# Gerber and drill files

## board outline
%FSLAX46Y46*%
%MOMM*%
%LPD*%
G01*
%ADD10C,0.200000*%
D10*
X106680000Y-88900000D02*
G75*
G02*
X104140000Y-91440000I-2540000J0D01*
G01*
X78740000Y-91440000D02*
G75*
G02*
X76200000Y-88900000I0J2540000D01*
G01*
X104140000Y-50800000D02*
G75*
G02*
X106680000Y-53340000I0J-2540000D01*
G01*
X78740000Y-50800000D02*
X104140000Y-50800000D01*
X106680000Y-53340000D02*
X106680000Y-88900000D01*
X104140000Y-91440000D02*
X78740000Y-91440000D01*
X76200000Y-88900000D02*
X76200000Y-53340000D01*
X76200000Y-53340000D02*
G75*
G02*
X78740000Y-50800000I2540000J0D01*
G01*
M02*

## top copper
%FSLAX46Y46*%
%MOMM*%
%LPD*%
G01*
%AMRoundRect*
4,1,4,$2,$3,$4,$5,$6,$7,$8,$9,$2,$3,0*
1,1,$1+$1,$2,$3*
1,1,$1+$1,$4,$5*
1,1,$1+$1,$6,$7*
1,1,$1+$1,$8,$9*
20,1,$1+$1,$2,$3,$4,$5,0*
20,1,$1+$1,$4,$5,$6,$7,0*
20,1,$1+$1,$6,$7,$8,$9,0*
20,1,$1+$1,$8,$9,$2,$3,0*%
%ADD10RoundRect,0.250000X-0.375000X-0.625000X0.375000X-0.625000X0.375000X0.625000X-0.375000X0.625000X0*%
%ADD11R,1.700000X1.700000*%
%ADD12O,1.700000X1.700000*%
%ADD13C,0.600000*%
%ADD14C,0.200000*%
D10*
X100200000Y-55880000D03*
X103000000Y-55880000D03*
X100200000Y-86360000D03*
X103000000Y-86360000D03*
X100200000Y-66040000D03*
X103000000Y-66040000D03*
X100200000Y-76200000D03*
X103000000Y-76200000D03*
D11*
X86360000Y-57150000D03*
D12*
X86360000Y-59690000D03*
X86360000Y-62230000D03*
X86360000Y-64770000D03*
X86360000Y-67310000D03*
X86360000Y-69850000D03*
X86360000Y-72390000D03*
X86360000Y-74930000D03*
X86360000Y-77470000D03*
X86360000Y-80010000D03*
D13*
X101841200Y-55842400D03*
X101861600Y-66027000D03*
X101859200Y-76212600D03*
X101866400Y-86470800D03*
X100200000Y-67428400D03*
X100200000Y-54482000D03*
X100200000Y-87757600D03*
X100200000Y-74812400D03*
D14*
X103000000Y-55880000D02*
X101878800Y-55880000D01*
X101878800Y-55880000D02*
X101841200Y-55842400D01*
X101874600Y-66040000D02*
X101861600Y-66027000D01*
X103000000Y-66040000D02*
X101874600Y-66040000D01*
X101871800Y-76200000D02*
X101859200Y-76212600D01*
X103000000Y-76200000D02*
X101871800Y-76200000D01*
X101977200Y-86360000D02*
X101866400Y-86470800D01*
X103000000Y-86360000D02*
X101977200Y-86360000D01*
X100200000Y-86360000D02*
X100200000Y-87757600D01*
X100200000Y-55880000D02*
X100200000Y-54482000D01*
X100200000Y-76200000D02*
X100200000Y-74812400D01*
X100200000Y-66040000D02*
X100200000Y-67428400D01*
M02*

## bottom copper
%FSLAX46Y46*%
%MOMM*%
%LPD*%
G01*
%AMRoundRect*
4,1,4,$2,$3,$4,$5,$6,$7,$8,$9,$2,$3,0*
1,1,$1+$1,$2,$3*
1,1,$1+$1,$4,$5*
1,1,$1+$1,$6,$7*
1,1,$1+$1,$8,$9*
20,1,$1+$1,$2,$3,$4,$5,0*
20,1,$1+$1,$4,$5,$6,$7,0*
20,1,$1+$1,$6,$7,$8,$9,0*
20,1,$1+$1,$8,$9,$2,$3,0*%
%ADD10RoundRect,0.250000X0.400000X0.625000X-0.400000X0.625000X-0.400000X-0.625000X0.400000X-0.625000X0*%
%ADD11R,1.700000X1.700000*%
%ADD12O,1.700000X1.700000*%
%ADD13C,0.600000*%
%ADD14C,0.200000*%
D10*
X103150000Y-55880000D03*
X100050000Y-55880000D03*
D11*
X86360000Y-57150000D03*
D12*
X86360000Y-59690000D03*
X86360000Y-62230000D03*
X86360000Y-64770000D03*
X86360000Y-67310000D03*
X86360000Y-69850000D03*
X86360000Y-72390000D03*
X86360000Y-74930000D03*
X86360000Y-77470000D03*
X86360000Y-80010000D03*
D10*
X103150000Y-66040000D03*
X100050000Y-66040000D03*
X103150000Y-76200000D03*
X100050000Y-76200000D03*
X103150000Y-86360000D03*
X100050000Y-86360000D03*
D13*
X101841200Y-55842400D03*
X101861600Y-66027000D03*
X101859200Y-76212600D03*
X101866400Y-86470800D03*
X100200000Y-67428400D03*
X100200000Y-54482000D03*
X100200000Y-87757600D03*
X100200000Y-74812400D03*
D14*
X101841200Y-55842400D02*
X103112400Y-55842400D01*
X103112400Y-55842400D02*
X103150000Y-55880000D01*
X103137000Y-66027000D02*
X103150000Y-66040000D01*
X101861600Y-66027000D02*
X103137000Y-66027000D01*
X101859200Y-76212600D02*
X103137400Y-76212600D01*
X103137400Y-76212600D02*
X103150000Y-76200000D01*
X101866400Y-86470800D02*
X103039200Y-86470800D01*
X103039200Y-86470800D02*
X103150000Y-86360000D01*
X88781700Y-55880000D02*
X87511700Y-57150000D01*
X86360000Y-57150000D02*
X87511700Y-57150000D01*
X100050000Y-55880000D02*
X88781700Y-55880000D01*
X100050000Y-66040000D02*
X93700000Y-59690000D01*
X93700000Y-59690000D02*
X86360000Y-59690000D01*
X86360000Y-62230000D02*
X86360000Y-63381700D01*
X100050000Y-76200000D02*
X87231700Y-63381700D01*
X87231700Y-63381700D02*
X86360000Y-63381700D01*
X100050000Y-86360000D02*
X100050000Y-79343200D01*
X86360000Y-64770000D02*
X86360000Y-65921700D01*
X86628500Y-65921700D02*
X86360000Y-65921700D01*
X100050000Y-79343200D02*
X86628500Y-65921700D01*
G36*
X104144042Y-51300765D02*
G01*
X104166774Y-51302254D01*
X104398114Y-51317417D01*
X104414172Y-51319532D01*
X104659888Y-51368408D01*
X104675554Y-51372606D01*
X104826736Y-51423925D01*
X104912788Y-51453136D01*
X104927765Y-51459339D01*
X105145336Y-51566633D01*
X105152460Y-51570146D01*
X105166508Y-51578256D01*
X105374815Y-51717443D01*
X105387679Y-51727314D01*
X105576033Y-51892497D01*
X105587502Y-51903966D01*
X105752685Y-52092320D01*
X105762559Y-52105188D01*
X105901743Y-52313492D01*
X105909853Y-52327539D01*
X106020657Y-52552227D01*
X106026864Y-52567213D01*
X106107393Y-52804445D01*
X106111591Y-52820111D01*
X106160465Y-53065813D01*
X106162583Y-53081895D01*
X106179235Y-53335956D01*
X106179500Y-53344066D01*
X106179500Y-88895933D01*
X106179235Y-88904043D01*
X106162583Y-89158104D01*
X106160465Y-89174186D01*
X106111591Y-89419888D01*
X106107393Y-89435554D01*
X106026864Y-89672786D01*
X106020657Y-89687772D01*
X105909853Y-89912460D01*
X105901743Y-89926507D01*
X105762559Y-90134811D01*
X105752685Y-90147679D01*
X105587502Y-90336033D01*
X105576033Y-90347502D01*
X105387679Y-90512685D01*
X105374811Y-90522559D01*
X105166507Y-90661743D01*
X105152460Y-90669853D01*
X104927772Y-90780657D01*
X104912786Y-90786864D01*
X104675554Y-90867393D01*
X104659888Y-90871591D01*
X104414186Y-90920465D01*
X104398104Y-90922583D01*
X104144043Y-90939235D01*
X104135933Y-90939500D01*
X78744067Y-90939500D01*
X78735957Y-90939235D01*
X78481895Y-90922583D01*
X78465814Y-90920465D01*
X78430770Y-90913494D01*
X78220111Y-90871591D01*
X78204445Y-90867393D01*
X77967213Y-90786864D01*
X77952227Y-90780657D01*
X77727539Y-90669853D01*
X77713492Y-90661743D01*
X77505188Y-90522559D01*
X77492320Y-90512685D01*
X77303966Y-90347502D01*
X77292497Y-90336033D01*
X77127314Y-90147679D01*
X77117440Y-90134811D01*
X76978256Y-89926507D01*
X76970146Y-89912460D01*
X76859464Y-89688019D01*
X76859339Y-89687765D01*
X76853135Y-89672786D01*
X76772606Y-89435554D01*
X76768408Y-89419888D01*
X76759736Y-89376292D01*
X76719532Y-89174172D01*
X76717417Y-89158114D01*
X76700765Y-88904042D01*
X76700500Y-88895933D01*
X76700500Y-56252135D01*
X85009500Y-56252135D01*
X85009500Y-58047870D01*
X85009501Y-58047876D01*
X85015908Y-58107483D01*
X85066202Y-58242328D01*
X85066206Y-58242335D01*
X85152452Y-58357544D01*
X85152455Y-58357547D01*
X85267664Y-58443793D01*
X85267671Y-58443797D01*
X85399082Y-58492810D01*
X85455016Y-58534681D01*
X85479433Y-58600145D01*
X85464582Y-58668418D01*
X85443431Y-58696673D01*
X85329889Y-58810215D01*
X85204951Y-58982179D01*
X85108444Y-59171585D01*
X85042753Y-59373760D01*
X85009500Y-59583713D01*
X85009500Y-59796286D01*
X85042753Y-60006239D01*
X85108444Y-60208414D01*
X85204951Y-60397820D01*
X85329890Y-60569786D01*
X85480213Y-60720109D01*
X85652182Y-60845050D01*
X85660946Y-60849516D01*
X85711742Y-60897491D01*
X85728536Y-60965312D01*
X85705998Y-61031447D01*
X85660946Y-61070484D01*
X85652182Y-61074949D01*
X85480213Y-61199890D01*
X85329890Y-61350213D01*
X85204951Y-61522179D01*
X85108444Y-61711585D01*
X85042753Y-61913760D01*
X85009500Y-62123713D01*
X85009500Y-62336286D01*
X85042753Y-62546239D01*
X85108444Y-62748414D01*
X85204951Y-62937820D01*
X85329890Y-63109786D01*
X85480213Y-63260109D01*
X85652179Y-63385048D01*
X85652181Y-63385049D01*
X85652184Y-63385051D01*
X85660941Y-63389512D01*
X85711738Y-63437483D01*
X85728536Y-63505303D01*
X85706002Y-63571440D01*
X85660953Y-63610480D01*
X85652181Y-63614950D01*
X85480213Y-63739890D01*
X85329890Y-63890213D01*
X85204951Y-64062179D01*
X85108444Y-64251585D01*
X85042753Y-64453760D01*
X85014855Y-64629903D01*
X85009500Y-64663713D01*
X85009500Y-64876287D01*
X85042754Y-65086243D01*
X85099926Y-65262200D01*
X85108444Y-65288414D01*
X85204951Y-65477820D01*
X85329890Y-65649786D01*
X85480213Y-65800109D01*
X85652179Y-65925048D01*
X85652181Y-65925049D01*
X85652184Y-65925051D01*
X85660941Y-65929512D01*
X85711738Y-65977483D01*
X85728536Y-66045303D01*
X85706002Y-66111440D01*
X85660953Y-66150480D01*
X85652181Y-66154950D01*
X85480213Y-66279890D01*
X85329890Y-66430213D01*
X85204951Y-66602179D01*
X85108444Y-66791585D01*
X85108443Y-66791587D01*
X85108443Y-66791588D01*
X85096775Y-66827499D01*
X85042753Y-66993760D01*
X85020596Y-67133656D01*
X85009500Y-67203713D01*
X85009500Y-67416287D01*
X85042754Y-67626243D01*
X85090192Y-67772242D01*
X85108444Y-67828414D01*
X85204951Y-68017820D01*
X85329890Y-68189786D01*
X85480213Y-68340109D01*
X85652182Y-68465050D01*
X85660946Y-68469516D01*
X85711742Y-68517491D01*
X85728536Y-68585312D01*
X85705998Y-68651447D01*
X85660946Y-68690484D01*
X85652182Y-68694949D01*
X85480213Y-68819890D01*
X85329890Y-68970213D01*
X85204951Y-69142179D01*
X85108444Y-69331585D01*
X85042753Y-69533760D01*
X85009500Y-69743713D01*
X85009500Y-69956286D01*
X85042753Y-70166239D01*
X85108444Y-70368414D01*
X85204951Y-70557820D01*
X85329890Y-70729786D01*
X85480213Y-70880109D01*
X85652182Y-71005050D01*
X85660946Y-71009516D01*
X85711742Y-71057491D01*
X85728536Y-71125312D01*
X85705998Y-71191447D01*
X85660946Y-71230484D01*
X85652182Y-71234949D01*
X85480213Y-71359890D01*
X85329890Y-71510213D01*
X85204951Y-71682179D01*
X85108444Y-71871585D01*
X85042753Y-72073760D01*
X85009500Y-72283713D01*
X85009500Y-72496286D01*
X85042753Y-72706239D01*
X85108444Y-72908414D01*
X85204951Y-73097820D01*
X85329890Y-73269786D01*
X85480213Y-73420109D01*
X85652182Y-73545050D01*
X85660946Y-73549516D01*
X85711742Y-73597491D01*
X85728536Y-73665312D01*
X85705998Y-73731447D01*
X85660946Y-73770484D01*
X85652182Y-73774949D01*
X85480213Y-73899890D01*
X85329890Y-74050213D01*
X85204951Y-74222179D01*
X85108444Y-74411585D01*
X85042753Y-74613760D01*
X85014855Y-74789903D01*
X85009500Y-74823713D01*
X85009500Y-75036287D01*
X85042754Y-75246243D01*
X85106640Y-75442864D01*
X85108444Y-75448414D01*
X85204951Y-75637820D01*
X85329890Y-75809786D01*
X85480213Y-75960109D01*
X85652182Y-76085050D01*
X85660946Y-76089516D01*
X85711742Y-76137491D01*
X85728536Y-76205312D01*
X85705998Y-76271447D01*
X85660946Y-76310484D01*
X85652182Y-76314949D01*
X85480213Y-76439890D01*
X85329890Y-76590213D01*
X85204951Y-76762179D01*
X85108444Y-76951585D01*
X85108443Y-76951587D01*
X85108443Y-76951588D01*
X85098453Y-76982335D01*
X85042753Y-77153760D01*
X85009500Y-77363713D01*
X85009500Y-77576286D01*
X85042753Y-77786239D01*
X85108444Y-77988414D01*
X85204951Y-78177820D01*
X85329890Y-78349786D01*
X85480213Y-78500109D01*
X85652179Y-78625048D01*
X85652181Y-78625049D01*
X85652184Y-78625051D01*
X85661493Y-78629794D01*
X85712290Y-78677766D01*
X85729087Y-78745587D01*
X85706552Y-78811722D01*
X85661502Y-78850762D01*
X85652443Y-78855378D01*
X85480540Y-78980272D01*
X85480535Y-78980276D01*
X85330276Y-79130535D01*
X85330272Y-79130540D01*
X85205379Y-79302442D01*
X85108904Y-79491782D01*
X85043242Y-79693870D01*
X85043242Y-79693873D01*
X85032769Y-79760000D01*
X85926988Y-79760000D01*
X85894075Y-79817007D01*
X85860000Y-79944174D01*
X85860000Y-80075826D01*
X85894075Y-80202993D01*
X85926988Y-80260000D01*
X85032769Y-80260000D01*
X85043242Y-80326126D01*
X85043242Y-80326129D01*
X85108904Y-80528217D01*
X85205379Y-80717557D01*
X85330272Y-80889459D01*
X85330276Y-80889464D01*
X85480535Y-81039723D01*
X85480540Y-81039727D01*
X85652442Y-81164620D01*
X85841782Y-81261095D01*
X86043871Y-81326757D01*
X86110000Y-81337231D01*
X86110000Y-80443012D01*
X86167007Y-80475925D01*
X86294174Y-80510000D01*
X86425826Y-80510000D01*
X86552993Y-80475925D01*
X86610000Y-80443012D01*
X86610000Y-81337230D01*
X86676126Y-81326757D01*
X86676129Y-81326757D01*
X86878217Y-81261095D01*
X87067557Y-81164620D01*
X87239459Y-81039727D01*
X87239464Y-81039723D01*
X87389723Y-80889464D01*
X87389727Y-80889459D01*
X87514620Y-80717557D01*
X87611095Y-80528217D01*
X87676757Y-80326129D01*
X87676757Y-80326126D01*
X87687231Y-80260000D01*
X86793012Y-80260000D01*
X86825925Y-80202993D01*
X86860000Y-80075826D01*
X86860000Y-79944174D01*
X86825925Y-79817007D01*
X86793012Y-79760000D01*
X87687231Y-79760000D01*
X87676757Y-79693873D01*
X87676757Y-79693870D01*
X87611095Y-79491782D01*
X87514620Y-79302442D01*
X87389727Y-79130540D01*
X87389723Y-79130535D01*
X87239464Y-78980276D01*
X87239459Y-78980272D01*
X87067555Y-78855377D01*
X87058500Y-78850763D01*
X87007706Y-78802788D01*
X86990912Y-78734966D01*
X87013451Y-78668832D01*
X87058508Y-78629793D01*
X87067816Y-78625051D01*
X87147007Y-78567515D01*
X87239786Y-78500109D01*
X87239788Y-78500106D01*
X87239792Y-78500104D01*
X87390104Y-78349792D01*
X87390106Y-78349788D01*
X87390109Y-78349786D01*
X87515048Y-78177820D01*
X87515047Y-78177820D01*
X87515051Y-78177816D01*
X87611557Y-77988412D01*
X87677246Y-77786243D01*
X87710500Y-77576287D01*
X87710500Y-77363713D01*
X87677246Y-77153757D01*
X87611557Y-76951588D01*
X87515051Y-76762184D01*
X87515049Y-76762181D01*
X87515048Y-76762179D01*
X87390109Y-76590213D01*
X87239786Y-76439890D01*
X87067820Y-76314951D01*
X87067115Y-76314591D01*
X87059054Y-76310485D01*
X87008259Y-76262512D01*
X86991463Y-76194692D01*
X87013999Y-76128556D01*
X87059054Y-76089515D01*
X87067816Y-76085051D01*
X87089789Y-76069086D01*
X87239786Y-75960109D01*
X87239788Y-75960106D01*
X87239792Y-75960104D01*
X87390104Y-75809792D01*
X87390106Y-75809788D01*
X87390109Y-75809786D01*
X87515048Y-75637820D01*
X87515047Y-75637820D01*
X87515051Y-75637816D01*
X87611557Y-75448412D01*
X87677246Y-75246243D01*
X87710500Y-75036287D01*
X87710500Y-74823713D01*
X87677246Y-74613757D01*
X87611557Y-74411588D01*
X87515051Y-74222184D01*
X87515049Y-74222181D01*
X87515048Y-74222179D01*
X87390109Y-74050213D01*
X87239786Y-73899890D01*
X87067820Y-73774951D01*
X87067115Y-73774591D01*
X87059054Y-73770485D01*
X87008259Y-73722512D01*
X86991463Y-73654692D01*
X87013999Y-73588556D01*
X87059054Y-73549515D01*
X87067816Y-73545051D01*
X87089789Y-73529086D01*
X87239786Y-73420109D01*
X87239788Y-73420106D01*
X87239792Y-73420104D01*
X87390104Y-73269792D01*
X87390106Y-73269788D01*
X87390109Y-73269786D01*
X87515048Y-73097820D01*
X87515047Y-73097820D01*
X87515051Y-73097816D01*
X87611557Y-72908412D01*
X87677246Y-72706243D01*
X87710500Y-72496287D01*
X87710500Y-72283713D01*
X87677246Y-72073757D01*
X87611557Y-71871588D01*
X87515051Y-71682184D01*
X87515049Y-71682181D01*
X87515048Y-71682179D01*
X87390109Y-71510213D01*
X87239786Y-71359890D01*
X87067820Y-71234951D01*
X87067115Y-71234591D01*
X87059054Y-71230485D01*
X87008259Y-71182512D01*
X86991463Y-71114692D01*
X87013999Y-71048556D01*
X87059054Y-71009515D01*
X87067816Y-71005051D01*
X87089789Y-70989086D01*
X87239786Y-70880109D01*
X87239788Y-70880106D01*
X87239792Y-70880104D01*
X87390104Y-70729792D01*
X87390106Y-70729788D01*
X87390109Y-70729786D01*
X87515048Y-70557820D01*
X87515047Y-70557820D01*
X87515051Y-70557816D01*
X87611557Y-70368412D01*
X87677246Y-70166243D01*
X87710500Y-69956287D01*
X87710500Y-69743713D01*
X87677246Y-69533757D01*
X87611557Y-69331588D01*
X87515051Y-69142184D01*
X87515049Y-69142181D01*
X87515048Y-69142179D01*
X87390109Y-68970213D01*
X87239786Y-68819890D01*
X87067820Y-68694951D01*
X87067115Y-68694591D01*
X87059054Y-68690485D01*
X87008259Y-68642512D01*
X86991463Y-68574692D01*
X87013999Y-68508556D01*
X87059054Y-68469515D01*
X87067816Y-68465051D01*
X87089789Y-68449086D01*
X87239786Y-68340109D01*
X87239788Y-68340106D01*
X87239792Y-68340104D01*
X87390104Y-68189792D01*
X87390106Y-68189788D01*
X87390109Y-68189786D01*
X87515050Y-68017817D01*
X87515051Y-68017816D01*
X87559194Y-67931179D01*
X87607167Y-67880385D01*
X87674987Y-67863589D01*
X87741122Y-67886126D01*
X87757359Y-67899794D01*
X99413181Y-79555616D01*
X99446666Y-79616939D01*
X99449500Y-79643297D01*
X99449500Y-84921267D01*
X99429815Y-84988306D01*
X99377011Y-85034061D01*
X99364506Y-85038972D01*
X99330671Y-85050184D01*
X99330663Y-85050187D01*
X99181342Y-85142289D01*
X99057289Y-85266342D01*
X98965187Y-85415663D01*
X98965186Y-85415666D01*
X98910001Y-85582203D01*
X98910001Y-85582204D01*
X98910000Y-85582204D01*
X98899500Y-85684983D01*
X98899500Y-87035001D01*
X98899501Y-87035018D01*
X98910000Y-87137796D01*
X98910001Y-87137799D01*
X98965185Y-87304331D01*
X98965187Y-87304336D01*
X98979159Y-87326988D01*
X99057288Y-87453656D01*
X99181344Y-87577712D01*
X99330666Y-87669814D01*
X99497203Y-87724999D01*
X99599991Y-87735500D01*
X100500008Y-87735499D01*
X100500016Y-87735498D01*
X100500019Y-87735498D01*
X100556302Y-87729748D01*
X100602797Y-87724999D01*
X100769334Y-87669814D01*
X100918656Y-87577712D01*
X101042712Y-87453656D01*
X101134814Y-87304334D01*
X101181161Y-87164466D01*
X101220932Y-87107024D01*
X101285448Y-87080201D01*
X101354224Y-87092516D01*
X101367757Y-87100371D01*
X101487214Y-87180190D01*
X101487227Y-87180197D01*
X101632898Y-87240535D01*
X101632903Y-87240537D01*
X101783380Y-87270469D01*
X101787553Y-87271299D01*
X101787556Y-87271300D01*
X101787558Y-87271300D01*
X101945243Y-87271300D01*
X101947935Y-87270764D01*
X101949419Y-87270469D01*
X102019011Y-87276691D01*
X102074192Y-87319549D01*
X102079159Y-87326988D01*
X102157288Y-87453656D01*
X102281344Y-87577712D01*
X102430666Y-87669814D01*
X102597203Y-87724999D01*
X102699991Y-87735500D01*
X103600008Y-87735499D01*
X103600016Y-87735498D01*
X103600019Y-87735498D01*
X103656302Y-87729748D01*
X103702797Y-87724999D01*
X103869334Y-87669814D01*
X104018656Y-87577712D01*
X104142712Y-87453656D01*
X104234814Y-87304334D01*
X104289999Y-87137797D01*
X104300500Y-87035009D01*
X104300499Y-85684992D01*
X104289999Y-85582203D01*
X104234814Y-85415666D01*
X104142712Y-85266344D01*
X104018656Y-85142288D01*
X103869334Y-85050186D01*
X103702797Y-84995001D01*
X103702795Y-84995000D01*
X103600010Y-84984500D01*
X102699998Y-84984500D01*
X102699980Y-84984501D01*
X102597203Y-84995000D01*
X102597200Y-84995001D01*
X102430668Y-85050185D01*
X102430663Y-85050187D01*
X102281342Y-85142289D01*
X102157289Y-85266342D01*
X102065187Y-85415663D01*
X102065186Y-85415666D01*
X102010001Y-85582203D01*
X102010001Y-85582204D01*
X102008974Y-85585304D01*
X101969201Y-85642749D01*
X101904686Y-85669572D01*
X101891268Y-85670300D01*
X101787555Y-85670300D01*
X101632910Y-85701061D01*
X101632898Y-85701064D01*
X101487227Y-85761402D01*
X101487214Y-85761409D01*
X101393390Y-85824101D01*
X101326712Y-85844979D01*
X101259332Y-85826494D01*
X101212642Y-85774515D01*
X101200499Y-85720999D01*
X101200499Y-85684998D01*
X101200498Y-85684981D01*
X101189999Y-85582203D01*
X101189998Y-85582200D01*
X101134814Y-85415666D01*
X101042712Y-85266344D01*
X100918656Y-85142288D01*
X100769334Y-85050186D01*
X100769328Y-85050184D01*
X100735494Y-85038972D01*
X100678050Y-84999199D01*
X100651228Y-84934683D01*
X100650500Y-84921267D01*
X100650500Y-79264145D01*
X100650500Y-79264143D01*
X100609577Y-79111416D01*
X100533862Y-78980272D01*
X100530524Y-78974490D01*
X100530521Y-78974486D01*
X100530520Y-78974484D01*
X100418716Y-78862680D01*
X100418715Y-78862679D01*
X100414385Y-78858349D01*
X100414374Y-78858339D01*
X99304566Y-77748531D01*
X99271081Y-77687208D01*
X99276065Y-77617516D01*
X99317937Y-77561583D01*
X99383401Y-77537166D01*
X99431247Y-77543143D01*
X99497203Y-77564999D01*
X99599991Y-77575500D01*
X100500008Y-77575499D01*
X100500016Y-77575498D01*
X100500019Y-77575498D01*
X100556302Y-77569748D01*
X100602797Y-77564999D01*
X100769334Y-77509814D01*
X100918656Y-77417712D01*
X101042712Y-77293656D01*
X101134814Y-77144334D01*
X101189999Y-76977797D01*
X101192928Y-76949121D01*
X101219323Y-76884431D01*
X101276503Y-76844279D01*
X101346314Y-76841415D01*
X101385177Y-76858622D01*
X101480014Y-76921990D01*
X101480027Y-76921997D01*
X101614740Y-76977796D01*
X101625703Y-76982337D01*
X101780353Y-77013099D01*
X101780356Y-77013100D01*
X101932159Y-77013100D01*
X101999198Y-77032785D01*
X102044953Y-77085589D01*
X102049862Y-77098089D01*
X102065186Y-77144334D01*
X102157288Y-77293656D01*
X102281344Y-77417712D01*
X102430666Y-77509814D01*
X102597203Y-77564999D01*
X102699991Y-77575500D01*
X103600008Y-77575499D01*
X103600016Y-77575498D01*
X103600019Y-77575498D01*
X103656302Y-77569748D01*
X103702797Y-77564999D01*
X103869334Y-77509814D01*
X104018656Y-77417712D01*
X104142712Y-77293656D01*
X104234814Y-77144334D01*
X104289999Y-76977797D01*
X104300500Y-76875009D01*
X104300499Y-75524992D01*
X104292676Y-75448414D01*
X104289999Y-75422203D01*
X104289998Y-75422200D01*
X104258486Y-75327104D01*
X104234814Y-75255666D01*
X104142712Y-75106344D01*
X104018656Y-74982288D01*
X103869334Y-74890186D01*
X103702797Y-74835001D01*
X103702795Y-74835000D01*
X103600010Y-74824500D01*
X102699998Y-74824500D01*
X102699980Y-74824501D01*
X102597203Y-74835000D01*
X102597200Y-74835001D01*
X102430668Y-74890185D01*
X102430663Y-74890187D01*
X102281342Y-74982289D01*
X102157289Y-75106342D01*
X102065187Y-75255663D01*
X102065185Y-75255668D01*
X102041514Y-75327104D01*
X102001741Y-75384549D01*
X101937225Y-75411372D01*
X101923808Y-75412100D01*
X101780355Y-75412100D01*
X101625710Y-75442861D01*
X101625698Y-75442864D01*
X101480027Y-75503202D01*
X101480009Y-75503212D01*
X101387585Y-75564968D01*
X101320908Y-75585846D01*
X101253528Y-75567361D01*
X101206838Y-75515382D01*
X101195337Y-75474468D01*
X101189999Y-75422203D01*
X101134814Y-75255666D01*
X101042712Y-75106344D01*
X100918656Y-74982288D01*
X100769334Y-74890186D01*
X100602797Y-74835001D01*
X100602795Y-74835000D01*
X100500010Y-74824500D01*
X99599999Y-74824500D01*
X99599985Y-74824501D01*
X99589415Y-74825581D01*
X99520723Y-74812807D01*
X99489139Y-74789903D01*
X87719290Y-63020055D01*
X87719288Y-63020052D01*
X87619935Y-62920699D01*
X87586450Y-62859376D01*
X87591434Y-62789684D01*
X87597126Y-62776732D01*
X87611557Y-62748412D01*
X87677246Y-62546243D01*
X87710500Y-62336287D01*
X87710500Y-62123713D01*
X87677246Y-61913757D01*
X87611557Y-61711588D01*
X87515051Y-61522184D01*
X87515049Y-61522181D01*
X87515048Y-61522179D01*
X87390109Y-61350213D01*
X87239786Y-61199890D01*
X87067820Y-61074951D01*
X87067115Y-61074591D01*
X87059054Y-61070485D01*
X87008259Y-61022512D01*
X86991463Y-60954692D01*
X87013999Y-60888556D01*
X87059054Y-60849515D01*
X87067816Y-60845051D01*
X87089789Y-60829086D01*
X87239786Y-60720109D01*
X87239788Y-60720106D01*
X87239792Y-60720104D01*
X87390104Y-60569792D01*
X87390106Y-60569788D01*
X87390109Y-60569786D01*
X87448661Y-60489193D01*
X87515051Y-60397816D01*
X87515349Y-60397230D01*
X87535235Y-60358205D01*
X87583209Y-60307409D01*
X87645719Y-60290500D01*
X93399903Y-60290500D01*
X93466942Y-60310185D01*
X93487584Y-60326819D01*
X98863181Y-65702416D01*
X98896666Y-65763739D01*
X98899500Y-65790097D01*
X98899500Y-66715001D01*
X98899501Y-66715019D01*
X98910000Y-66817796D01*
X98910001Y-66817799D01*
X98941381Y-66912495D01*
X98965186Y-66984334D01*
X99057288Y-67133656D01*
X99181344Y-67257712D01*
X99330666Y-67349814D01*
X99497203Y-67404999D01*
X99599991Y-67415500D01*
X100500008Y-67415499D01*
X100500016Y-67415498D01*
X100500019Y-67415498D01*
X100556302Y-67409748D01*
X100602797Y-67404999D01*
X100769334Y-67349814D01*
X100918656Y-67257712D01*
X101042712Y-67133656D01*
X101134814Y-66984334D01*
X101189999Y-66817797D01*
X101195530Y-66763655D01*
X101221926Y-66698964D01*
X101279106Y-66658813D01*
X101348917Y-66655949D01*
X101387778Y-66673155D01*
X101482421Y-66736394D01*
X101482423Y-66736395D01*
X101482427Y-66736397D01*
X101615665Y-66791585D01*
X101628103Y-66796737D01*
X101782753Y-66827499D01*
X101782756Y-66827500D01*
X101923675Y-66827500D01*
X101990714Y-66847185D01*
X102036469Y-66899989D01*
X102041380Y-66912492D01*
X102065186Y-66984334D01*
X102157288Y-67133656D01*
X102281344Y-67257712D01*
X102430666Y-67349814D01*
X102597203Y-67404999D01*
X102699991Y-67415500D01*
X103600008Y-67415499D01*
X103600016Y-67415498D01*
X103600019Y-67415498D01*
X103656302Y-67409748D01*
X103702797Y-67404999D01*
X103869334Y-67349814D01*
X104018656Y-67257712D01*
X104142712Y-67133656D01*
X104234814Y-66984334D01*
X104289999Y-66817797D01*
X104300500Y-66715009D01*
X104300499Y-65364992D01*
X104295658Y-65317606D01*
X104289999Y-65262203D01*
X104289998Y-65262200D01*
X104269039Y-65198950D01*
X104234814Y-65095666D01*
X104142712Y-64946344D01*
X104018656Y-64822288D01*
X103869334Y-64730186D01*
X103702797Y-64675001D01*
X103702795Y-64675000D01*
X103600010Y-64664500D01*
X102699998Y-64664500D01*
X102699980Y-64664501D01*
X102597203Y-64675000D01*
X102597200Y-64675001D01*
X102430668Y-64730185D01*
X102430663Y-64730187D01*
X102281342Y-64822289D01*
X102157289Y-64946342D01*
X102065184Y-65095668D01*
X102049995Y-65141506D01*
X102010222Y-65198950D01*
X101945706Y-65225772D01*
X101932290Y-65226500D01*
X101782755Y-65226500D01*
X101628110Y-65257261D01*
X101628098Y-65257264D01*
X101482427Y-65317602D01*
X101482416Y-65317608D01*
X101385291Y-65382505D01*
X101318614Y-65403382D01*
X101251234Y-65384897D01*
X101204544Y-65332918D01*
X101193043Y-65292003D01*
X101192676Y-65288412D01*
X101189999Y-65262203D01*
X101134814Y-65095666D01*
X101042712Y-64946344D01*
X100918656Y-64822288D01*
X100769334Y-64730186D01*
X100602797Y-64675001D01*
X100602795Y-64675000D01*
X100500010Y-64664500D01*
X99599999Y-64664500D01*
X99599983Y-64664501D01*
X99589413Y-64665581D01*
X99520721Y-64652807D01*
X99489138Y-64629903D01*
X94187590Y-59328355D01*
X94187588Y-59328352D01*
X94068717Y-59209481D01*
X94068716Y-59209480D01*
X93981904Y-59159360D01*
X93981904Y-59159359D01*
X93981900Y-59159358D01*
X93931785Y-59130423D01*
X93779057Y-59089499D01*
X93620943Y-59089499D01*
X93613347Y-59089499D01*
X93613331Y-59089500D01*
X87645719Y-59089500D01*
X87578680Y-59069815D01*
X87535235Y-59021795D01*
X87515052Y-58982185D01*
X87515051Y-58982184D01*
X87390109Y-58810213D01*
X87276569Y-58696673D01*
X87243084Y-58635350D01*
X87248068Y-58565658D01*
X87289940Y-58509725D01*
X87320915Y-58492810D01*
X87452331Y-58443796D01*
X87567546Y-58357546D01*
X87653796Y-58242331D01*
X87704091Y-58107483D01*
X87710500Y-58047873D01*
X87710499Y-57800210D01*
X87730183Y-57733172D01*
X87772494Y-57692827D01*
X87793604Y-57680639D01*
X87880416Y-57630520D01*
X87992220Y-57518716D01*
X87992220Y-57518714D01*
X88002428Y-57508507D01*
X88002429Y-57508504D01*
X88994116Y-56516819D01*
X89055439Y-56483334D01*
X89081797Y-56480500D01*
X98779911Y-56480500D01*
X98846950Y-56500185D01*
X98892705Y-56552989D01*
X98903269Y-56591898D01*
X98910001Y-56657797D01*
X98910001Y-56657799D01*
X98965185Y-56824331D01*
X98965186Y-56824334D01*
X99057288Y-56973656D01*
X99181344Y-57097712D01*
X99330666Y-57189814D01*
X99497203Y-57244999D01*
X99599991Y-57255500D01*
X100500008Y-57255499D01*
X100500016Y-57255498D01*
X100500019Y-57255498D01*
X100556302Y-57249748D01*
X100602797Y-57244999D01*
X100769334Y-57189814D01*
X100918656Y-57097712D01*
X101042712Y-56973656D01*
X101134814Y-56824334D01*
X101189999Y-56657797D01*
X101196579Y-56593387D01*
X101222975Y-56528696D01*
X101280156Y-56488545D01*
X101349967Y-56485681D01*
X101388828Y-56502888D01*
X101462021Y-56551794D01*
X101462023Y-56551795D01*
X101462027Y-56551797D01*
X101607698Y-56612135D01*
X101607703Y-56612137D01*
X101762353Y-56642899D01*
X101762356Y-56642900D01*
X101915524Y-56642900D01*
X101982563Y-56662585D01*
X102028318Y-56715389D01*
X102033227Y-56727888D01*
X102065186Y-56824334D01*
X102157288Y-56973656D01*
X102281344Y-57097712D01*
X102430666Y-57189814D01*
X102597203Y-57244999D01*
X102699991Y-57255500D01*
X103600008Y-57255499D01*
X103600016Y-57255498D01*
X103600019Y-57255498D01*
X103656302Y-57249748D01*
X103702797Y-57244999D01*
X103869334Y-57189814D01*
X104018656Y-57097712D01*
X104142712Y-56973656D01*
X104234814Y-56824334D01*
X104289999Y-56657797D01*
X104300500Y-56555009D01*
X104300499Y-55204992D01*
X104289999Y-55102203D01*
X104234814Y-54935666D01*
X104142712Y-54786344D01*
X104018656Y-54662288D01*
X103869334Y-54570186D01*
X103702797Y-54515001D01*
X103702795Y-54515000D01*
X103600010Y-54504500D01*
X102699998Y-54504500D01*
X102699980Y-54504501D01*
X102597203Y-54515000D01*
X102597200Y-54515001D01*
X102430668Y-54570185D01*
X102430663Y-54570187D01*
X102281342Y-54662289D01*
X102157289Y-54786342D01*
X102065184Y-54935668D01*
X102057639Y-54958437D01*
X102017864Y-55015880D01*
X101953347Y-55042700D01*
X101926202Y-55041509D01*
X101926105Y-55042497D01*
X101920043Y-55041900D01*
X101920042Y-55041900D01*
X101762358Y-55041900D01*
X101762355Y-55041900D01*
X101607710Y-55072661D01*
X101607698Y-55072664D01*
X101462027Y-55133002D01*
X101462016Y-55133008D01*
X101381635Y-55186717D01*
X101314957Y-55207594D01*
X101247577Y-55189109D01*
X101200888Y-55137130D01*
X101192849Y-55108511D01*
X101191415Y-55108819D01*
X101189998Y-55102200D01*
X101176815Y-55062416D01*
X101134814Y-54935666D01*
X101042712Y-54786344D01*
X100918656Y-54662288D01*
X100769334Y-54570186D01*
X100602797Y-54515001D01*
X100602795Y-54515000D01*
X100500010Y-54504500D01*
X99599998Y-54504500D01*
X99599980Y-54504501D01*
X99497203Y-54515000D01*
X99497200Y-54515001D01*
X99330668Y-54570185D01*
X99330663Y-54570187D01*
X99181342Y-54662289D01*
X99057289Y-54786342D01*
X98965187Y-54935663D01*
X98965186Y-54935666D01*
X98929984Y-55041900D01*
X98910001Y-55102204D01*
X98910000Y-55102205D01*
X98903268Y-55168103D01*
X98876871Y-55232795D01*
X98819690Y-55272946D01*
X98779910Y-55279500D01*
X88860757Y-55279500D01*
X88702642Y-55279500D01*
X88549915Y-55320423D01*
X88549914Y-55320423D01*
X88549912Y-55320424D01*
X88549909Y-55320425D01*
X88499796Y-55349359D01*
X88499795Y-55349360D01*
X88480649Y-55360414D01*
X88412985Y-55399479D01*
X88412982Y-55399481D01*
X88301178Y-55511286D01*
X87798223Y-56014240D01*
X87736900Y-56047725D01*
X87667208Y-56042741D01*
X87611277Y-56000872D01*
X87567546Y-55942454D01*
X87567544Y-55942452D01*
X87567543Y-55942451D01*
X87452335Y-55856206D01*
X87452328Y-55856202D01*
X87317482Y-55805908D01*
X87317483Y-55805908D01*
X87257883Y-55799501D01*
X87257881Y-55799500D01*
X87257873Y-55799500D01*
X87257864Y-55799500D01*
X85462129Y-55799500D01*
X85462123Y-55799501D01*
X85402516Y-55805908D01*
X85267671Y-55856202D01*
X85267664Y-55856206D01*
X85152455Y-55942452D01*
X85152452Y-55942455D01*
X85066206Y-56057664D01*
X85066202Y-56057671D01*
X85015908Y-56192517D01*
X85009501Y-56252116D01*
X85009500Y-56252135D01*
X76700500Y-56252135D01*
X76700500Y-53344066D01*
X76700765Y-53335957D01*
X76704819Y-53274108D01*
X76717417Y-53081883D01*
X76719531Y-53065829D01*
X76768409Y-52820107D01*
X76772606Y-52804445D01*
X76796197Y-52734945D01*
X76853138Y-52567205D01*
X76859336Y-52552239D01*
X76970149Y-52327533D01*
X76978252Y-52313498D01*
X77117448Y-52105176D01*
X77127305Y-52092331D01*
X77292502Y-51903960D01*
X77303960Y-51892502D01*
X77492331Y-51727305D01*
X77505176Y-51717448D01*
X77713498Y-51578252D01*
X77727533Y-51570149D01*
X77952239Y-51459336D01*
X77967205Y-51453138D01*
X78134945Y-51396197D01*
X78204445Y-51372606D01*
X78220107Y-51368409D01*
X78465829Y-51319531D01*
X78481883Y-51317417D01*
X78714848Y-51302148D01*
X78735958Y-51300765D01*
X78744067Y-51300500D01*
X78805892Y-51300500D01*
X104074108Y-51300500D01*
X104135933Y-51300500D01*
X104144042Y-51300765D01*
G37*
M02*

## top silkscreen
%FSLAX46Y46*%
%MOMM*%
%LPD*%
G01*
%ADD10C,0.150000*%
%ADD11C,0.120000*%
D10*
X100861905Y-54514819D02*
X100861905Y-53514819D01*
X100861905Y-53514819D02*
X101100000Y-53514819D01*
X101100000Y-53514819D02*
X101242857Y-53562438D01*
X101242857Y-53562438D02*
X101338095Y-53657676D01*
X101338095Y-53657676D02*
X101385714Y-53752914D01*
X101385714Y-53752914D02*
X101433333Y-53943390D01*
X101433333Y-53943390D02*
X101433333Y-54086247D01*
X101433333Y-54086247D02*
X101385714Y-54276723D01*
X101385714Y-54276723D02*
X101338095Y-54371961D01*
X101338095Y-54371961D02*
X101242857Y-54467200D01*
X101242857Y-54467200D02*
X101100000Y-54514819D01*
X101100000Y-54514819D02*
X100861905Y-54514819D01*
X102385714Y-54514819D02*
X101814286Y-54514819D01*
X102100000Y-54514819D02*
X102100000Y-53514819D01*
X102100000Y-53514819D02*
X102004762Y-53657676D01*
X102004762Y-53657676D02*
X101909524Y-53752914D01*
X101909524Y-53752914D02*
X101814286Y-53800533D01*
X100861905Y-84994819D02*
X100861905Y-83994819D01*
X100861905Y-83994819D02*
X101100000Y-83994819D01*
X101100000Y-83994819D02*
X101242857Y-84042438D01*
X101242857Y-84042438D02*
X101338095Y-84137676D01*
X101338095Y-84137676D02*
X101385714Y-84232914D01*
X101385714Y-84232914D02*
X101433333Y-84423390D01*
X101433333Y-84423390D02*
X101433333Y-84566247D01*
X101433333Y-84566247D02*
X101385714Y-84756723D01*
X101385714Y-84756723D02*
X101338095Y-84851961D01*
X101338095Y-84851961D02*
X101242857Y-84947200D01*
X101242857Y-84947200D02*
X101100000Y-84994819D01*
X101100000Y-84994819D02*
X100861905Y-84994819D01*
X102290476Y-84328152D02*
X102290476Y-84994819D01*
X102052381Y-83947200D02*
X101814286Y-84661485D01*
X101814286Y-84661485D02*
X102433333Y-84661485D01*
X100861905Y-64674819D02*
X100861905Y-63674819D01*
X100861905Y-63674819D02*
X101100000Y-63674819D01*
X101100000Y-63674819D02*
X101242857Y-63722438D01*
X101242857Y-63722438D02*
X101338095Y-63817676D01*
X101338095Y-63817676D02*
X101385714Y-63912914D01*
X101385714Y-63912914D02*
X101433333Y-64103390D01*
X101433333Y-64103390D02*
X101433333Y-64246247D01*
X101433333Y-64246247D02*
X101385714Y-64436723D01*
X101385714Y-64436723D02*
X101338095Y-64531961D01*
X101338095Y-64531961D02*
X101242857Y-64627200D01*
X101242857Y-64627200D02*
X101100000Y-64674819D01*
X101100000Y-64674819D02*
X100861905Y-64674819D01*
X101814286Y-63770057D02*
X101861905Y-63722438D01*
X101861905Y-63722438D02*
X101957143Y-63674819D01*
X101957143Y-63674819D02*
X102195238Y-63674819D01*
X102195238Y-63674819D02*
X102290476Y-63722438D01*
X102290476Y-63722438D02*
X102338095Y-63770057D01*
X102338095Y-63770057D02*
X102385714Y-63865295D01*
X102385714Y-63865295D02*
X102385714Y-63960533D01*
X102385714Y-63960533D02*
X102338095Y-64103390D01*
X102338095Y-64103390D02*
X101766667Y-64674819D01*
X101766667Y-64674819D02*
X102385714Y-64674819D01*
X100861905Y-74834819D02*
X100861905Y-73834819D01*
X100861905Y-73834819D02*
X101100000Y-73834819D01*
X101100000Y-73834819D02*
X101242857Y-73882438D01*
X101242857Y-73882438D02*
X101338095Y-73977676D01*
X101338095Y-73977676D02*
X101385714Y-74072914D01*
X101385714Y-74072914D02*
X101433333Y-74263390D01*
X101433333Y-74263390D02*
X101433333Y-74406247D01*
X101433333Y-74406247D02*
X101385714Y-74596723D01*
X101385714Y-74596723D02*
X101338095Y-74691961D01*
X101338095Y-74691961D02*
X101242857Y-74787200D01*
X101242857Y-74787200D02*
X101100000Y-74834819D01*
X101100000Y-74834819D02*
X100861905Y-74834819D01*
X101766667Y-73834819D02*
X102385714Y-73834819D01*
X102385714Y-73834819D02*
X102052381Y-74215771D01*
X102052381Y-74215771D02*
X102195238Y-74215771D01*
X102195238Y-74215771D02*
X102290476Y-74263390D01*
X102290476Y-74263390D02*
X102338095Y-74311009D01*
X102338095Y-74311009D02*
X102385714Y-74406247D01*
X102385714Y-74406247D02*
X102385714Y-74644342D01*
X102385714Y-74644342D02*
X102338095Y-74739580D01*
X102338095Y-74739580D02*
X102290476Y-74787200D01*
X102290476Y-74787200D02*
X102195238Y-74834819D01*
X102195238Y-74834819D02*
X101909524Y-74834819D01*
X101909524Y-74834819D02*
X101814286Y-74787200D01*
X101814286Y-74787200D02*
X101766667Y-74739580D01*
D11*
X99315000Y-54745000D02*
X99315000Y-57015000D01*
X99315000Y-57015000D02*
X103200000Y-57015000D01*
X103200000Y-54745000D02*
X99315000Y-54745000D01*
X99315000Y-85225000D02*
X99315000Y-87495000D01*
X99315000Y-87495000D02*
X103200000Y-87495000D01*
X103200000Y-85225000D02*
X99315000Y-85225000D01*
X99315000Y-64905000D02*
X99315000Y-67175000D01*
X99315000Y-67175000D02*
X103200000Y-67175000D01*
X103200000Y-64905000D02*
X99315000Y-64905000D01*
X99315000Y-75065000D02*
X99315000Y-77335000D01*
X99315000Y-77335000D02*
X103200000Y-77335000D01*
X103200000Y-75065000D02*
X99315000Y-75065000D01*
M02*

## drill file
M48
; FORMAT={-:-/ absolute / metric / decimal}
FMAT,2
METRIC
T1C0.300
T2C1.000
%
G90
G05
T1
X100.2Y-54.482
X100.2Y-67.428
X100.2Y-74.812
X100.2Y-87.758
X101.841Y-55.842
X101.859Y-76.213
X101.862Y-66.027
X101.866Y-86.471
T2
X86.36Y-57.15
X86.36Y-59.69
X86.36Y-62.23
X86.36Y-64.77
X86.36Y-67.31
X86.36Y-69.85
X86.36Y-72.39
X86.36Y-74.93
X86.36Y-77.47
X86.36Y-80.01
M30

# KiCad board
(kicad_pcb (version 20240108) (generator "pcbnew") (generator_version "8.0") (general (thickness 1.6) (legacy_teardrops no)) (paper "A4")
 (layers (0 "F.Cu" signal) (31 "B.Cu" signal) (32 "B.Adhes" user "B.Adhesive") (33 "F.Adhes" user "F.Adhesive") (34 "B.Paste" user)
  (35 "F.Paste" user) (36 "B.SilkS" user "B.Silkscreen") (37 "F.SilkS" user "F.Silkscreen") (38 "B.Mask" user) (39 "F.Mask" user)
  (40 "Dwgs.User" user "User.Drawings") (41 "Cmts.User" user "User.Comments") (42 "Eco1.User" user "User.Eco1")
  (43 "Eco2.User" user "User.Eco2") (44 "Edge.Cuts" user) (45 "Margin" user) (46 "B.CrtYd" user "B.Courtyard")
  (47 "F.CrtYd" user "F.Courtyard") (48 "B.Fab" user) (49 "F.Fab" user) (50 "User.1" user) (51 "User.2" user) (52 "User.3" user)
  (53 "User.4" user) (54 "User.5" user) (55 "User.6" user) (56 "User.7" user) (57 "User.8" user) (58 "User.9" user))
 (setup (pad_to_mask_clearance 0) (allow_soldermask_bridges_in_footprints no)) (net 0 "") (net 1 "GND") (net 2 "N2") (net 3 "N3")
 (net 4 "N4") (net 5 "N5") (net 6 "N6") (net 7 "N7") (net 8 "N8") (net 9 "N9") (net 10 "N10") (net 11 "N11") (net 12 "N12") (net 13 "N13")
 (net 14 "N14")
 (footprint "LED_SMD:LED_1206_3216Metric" (layer "F.Cu") (at 101.6 55.88)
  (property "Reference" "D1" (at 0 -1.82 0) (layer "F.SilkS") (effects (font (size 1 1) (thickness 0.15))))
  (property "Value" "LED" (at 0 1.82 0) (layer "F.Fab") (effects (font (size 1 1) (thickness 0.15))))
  (fp_line (start -2.285 -1.135) (end -2.285 1.135) (stroke (width 0.12) (type solid)) (layer "F.SilkS"))
  (fp_line (start -2.285 1.135) (end 1.6 1.135) (stroke (width 0.12) (type solid)) (layer "F.SilkS"))
  (fp_line (start 1.6 -1.135) (end -2.285 -1.135) (stroke (width 0.12) (type solid)) (layer "F.SilkS"))
  (pad "1" smd roundrect (at -1.4 0) (size 1.25 1.75) (layers "F.Cu" "F.Paste" "F.Mask") (roundrect_rratio 0.2) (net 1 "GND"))
  (pad "2" smd roundrect (at 1.4 0) (size 1.25 1.75) (layers "F.Cu" "F.Paste" "F.Mask") (roundrect_rratio 0.2) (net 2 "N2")))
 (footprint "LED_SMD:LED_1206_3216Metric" (layer "F.Cu") (at 101.6 86.36)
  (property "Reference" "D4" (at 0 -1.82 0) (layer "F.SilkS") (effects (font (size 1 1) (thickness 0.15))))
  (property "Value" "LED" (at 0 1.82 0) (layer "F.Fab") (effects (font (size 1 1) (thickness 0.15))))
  (fp_line (start -2.285 -1.135) (end -2.285 1.135) (stroke (width 0.12) (type solid)) (layer "F.SilkS"))
  (fp_line (start -2.285 1.135) (end 1.6 1.135) (stroke (width 0.12) (type solid)) (layer "F.SilkS"))
  (fp_line (start 1.6 -1.135) (end -2.285 -1.135) (stroke (width 0.12) (type solid)) (layer "F.SilkS"))
  (pad "1" smd roundrect (at -1.4 0) (size 1.25 1.75) (layers "F.Cu" "F.Paste" "F.Mask") (roundrect_rratio 0.2) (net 1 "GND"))
  (pad "2" smd roundrect (at 1.4 0) (size 1.25 1.75) (layers "F.Cu" "F.Paste" "F.Mask") (roundrect_rratio 0.2) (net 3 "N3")))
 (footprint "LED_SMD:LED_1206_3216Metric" (layer "F.Cu") (at 101.6 66.04)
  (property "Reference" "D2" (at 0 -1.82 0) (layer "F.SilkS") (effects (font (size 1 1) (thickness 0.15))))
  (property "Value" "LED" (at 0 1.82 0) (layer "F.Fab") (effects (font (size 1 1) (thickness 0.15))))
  (fp_line (start -2.285 -1.135) (end -2.285 1.135) (stroke (width 0.12) (type solid)) (layer "F.SilkS"))
  (fp_line (start -2.285 1.135) (end 1.6 1.135) (stroke (width 0.12) (type solid)) (layer "F.SilkS"))
  (fp_line (start 1.6 -1.135) (end -2.285 -1.135) (stroke (width 0.12) (type solid)) (layer "F.SilkS"))
  (pad "1" smd roundrect (at -1.4 0) (size 1.25 1.75) (layers "F.Cu" "F.Paste" "F.Mask") (roundrect_rratio 0.2) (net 1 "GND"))
  (pad "2" smd roundrect (at 1.4 0) (size 1.25 1.75) (layers "F.Cu" "F.Paste" "F.Mask") (roundrect_rratio 0.2) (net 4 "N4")))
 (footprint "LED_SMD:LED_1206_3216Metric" (layer "F.Cu") (at 101.6 76.2)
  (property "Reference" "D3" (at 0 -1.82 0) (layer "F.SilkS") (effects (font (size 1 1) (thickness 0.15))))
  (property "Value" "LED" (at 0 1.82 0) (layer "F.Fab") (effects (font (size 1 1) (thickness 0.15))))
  (fp_line (start -2.285 -1.135) (end -2.285 1.135) (stroke (width 0.12) (type solid)) (layer "F.SilkS"))
  (fp_line (start -2.285 1.135) (end 1.6 1.135) (stroke (width 0.12) (type solid)) (layer "F.SilkS"))
  (fp_line (start 1.6 -1.135) (end -2.285 -1.135) (stroke (width 0.12) (type solid)) (layer "F.SilkS"))
  (pad "1" smd roundrect (at -1.4 0) (size 1.25 1.75) (layers "F.Cu" "F.Paste" "F.Mask") (roundrect_rratio 0.2) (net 1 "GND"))
  (pad "2" smd roundrect (at 1.4 0) (size 1.25 1.75) (layers "F.Cu" "F.Paste" "F.Mask") (roundrect_rratio 0.2) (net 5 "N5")))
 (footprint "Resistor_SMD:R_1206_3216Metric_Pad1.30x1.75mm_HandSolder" (layer "B.Cu") (at 101.6 55.88 180)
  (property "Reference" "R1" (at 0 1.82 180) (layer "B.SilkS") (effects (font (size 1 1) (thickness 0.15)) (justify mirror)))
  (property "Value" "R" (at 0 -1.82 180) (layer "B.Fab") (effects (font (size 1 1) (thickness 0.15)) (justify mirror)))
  (pad "1" smd roundrect (at -1.55 0 180) (size 1.3 1.75) (layers "B.Cu" "B.Paste" "B.Mask") (roundrect_rratio 0.192308) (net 2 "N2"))
  (pad "2" smd roundrect (at 1.55 0 180) (size 1.3 1.75) (layers "B.Cu" "B.Paste" "B.Mask") (roundrect_rratio 0.192308) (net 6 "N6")))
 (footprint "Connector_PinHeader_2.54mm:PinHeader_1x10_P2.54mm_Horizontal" (layer "B.Cu") (at 86.36 57.15 180)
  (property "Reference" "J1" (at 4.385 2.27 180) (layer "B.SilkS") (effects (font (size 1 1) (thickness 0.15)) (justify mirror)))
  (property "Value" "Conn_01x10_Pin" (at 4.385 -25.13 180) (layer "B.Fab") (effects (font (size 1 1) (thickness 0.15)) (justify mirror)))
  (pad "1" thru_hole rect (at 0 0 180) (size 1.7 1.7) (drill 1) (layers "*.Cu" "*.Mask") (remove_unused_layers no) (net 6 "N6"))
  (pad "2" thru_hole oval (at 0 -2.54 180) (size 1.7 1.7) (drill 1) (layers "*.Cu" "*.Mask") (remove_unused_layers no) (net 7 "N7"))
  (pad "3" thru_hole oval (at 0 -5.08 180) (size 1.7 1.7) (drill 1) (layers "*.Cu" "*.Mask") (remove_unused_layers no) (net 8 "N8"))
  (pad "4" thru_hole oval (at 0 -7.62 180) (size 1.7 1.7) (drill 1) (layers "*.Cu" "*.Mask") (remove_unused_layers no) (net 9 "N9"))
  (pad "5" thru_hole oval (at 0 -10.16 180) (size 1.7 1.7) (drill 1) (layers "*.Cu" "*.Mask") (remove_unused_layers no) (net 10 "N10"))
  (pad "6" thru_hole oval (at 0 -12.7 180) (size 1.7 1.7) (drill 1) (layers "*.Cu" "*.Mask") (remove_unused_layers no) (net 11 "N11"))
  (pad "7" thru_hole oval (at 0 -15.24 180) (size 1.7 1.7) (drill 1) (layers "*.Cu" "*.Mask") (remove_unused_layers no) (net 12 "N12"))
  (pad "8" thru_hole oval (at 0 -17.78 180) (size 1.7 1.7) (drill 1) (layers "*.Cu" "*.Mask") (remove_unused_layers no) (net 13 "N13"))
  (pad "9" thru_hole oval (at 0 -20.32 180) (size 1.7 1.7) (drill 1) (layers "*.Cu" "*.Mask") (remove_unused_layers no) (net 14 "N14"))
  (pad "10" thru_hole oval (at 0 -22.86 180) (size 1.7 1.7) (drill 1) (layers "*.Cu" "*.Mask") (remove_unused_layers no) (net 1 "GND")))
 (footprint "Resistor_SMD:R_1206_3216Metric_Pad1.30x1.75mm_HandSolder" (layer "B.Cu") (at 101.6 66.04 180)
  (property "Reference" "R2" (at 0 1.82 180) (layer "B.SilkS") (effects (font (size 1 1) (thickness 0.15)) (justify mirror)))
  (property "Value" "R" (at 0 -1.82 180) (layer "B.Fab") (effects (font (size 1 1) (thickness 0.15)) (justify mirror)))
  (pad "1" smd roundrect (at -1.55 0 180) (size 1.3 1.75) (layers "B.Cu" "B.Paste" "B.Mask") (roundrect_rratio 0.192308) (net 4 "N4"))
  (pad "2" smd roundrect (at 1.55 0 180) (size 1.3 1.75) (layers "B.Cu" "B.Paste" "B.Mask") (roundrect_rratio 0.192308) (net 7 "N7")))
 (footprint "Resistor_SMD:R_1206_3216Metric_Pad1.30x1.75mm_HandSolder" (layer "B.Cu") (at 101.6 76.2 180)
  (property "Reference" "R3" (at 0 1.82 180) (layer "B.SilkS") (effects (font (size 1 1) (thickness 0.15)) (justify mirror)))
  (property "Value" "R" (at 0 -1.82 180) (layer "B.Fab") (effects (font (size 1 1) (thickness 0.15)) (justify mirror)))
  (pad "1" smd roundrect (at -1.55 0 180) (size 1.3 1.75) (layers "B.Cu" "B.Paste" "B.Mask") (roundrect_rratio 0.192308) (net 5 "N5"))
  (pad "2" smd roundrect (at 1.55 0 180) (size 1.3 1.75) (layers "B.Cu" "B.Paste" "B.Mask") (roundrect_rratio 0.192308) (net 8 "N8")))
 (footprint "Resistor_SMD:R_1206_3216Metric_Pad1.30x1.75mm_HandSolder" (layer "B.Cu") (at 101.6 86.36 180)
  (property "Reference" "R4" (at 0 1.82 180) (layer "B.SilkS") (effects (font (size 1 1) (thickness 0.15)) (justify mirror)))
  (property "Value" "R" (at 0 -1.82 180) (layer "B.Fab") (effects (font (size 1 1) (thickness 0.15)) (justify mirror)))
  (pad "1" smd roundrect (at -1.55 0 180) (size 1.3 1.75) (layers "B.Cu" "B.Paste" "B.Mask") (roundrect_rratio 0.192308) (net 3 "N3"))
  (pad "2" smd roundrect (at 1.55 0 180) (size 1.3 1.75) (layers "B.Cu" "B.Paste" "B.Mask") (roundrect_rratio 0.192308) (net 9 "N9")))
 (gr_arc (start 106.68 88.9) (mid 105.936051 90.696051) (end 104.14 91.44) (stroke (width 0.2) (type default)) (layer "Edge.Cuts"))
 (gr_arc (start 78.74 91.44) (mid 76.943949 90.696051) (end 76.2 88.9) (stroke (width 0.2) (type default)) (layer "Edge.Cuts"))
 (gr_arc (start 104.14 50.8) (mid 105.936051 51.543949) (end 106.68 53.34) (stroke (width 0.2) (type default)) (layer "Edge.Cuts"))
 (gr_line (start 78.74 50.8) (end 104.14 50.8) (stroke (width 0.2) (type default)) (layer "Edge.Cuts"))
 (gr_line (start 106.68 53.34) (end 106.68 88.9) (stroke (width 0.2) (type default)) (layer "Edge.Cuts"))
 (gr_line (start 104.14 91.44) (end 78.74 91.44) (stroke (width 0.2) (type default)) (layer "Edge.Cuts"))
 (gr_line (start 76.2 88.9) (end 76.2 53.34) (stroke (width 0.2) (type default)) (layer "Edge.Cuts"))
 (gr_arc (start 76.2 53.34) (mid 76.943949 51.543949) (end 78.74 50.8) (stroke (width 0.2) (type default)) (layer "Edge.Cuts"))
 (segment (start 103 55.88) (end 101.8788 55.88) (width 0.2) (layer "F.Cu") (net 2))
 (segment (start 101.8788 55.88) (end 101.8412 55.8424) (width 0.2) (layer "F.Cu") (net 2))
 (via (at 101.8412 55.8424) (size 0.6) (drill 0.3) (layers "F.Cu" "B.Cu") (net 2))
 (segment (start 101.8412 55.8424) (end 103.1124 55.8424) (width 0.2) (layer "B.Cu") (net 2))
 (segment (start 103.1124 55.8424) (end 103.15 55.88) (width 0.2) (layer "B.Cu") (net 2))
 (segment (start 101.8746 66.04) (end 101.8616 66.027) (width 0.2) (layer "F.Cu") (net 4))
 (segment (start 103 66.04) (end 101.8746 66.04) (width 0.2) (layer "F.Cu") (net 4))
 (via (at 101.8616 66.027) (size 0.6) (drill 0.3) (layers "F.Cu" "B.Cu") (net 4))
 (segment (start 103.137 66.027) (end 103.15 66.04) (width 0.2) (layer "B.Cu") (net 4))
 (segment (start 101.8616 66.027) (end 103.137 66.027) (width 0.2) (layer "B.Cu") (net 4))
 (segment (start 101.8718 76.2) (end 101.8592 76.2126) (width 0.2) (layer "F.Cu") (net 5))
 (segment (start 103 76.2) (end 101.8718 76.2) (width 0.2) (layer "F.Cu") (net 5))
 (via (at 101.8592 76.2126) (size 0.6) (drill 0.3) (layers "F.Cu" "B.Cu") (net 5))
 (segment (start 101.8592 76.2126) (end 103.1374 76.2126) (width 0.2) (layer "B.Cu") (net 5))
 (segment (start 103.1374 76.2126) (end 103.15 76.2) (width 0.2) (layer "B.Cu") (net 5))
 (segment (start 101.9772 86.36) (end 101.8664 86.4708) (width 0.2) (layer "F.Cu") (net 3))
 (segment (start 103 86.36) (end 101.9772 86.36) (width 0.2) (layer "F.Cu") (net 3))
 (via (at 101.8664 86.4708) (size 0.6) (drill 0.3) (layers "F.Cu" "B.Cu") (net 3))
 (segment (start 101.8664 86.4708) (end 103.0392 86.4708) (width 0.2) (layer "B.Cu") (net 3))
 (segment (start 103.0392 86.4708) (end 103.15 86.36) (width 0.2) (layer "B.Cu") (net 3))
 (segment (start 88.7817 55.88) (end 87.5117 57.15) (width 0.2) (layer "B.Cu") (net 6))
 (segment (start 86.36 57.15) (end 87.5117 57.15) (width 0.2) (layer "B.Cu") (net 6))
 (segment (start 100.05 55.88) (end 88.7817 55.88) (width 0.2) (layer "B.Cu") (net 6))
 (segment (start 100.05 66.04) (end 93.7 59.69) (width 0.2) (layer "B.Cu") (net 7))
 (segment (start 93.7 59.69) (end 86.36 59.69) (width 0.2) (layer "B.Cu") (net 7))
 (segment (start 86.36 62.23) (end 86.36 63.3817) (width 0.2) (layer "B.Cu") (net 8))
 (segment (start 100.05 76.2) (end 87.2317 63.3817) (width 0.2) (layer "B.Cu") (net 8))
 (segment (start 87.2317 63.3817) (end 86.36 63.3817) (width 0.2) (layer "B.Cu") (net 8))
 (segment (start 100.05 86.36) (end 100.05 79.3432) (width 0.2) (layer "B.Cu") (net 9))
 (segment (start 86.36 64.77) (end 86.36 65.9217) (width 0.2) (layer "B.Cu") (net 9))
 (segment (start 86.6285 65.9217) (end 86.36 65.9217) (width 0.2) (layer "B.Cu") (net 9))
 (segment (start 100.05 79.3432) (end 86.6285 65.9217) (width 0.2) (layer "B.Cu") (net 9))
 (segment (start 100.2 86.36) (end 100.2 87.7576) (width 0.2) (layer "F.Cu") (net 1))
 (segment (start 100.2 55.88) (end 100.2 54.482) (width 0.2) (layer "F.Cu") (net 1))
 (segment (start 100.2 76.2) (end 100.2 74.8124) (width 0.2) (layer "F.Cu") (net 1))
 (segment (start 100.2 66.04) (end 100.2 67.4284) (width 0.2) (layer "F.Cu") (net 1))
 (via (at 100.2 67.4284) (size 0.6) (drill 0.3) (layers "F.Cu" "B.Cu") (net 1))
 (via (at 100.2 54.482) (size 0.6) (drill 0.3) (layers "F.Cu" "B.Cu") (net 1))
 (via (at 100.2 87.7576) (size 0.6) (drill 0.3) (layers "F.Cu" "B.Cu") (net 1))
 (via (at 100.2 74.8124) (size 0.6) (drill 0.3) (layers "F.Cu" "B.Cu") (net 1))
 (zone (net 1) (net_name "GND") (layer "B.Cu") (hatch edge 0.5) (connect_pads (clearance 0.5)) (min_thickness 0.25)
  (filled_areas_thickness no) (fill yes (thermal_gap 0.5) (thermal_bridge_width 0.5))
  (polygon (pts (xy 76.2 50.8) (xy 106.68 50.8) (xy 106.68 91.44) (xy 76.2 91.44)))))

